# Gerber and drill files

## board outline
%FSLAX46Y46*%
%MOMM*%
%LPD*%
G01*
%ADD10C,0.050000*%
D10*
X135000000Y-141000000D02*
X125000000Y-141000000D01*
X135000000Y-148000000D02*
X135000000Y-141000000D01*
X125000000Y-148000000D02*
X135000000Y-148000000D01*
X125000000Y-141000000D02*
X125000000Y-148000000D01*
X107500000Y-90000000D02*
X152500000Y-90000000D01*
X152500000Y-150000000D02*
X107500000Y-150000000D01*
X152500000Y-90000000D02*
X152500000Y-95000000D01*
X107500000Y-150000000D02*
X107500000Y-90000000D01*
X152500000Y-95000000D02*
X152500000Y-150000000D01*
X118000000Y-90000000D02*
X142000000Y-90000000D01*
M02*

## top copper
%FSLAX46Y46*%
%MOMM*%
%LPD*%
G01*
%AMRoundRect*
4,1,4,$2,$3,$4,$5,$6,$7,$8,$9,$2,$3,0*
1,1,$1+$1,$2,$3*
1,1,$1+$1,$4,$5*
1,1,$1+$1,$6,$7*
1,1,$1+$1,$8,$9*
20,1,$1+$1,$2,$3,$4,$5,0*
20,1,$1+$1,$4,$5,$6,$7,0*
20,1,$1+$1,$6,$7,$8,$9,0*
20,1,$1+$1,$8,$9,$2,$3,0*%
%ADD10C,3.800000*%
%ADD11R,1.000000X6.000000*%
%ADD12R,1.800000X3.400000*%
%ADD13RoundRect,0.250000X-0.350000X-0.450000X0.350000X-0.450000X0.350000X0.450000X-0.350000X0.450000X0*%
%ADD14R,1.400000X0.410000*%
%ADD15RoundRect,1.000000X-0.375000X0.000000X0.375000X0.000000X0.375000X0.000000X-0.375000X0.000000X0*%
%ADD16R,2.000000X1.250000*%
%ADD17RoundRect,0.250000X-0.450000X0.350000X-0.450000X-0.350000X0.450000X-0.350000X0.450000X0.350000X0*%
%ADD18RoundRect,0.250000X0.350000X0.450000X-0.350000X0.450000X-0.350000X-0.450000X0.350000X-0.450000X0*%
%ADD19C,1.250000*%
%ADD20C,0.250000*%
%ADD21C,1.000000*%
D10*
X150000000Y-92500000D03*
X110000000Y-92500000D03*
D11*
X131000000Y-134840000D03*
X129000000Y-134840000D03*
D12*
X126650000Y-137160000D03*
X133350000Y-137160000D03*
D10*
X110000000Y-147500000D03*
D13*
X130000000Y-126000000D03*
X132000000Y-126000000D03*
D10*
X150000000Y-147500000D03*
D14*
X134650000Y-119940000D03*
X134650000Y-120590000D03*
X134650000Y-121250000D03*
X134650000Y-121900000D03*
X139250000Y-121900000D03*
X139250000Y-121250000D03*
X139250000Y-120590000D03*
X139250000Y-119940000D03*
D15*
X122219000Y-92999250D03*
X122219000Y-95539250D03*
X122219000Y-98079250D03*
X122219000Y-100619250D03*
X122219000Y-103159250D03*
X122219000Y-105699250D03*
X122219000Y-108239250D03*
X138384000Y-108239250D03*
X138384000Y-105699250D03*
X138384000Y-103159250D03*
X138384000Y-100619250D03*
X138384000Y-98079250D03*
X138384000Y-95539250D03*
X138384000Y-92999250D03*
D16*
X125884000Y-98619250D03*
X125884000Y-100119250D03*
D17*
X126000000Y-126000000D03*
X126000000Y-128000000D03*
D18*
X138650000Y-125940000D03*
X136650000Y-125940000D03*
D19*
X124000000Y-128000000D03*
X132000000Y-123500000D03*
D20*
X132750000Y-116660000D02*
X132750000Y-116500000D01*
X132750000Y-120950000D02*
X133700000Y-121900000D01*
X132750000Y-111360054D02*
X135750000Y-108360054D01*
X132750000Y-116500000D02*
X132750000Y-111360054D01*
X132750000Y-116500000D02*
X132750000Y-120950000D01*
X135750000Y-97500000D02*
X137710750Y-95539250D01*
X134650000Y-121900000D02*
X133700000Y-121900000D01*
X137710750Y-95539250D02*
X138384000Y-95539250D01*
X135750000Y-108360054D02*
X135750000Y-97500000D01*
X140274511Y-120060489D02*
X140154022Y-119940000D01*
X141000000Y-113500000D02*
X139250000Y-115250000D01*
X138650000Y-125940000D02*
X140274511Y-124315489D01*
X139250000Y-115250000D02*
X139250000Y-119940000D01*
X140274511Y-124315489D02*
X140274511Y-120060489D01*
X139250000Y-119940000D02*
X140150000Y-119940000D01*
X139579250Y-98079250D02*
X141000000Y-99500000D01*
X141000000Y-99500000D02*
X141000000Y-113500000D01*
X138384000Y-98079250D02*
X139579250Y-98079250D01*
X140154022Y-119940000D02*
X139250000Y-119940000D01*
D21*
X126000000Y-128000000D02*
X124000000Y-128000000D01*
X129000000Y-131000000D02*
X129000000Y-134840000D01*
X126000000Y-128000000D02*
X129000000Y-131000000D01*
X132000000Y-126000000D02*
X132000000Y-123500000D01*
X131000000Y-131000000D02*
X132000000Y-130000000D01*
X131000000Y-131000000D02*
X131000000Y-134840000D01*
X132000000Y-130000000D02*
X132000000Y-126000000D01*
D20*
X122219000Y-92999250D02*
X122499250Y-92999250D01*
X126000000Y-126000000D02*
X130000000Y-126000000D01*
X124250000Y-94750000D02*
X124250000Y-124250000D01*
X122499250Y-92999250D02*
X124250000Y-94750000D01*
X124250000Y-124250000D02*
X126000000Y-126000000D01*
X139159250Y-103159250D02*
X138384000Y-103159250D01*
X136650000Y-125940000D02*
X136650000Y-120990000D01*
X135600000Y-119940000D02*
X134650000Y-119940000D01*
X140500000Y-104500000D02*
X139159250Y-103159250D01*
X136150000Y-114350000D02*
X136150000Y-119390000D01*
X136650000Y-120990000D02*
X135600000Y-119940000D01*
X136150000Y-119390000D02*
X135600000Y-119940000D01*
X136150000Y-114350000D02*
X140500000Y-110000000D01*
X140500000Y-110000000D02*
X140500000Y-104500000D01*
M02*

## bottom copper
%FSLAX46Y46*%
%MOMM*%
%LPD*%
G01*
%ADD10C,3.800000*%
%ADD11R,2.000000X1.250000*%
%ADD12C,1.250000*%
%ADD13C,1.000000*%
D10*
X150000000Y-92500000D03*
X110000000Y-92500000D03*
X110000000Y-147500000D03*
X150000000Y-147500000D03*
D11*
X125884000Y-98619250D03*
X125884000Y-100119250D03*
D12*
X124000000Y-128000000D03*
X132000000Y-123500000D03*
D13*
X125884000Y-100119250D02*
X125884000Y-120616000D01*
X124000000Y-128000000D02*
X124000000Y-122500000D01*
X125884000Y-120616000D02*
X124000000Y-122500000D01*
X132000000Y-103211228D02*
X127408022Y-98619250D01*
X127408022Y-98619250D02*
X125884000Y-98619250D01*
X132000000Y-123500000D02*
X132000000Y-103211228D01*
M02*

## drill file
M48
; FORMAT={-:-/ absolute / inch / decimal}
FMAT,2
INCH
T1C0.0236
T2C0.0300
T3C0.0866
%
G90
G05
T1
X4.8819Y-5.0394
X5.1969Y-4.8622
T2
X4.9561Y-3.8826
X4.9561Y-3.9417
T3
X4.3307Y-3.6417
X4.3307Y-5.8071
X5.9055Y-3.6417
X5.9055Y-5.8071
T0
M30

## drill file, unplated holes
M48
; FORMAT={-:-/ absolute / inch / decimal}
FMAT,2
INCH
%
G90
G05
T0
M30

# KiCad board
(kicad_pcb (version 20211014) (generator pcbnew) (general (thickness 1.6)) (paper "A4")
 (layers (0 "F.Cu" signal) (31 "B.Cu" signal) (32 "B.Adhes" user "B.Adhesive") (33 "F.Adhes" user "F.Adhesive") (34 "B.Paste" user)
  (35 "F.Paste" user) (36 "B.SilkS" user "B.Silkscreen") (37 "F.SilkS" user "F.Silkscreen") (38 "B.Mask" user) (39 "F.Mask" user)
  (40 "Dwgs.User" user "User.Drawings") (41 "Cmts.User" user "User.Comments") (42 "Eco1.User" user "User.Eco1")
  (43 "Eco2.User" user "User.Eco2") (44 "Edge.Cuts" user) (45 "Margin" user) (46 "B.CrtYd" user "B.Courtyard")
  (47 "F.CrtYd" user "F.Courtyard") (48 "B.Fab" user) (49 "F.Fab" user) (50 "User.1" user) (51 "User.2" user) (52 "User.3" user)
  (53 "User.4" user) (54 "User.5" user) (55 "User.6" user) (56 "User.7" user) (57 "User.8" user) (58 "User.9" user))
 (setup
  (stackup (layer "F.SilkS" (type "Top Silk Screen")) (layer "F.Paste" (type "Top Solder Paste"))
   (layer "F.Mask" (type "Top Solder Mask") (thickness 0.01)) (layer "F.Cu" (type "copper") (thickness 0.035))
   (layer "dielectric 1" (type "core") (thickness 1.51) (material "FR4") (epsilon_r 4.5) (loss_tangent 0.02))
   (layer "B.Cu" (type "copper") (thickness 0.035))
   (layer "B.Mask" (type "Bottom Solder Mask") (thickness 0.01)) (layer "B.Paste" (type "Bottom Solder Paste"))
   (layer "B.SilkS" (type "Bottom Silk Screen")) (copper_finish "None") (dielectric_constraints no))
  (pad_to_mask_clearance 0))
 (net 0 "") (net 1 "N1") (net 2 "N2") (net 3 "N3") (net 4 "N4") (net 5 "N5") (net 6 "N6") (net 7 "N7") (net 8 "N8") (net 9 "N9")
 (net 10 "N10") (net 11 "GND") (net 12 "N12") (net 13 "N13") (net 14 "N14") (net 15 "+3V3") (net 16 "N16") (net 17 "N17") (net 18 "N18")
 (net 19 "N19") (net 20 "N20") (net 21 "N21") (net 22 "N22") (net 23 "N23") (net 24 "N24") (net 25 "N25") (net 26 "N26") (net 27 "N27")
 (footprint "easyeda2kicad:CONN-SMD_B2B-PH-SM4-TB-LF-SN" (layer "F.Cu") (at 130 136)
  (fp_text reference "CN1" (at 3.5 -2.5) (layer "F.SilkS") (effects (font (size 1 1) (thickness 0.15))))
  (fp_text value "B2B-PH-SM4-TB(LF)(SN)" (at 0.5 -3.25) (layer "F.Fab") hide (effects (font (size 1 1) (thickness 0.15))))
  (pad "1" smd rect locked (at 1 -1.16) (size 1 6) (layers "F.Cu" "F.Paste" "F.Mask") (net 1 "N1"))
  (pad "2" smd rect locked (at -1 -1.16) (size 1 6) (layers "F.Cu" "F.Paste" "F.Mask") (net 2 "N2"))
  (pad "3" smd rect locked (at -3.35 1.16) (size 1.8 3.4) (layers "F.Cu" "F.Paste" "F.Mask") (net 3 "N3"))
  (pad "4" smd rect locked (at 3.35 1.16) (size 1.8 3.4) (layers "F.Cu" "F.Paste" "F.Mask") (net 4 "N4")))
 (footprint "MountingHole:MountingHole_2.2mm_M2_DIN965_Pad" (layer "F.Cu") (at 110 147.5)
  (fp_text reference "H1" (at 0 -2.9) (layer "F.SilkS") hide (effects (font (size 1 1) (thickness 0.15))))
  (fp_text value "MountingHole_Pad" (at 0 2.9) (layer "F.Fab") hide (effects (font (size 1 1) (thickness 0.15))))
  (pad "1" thru_hole circle (at 0 0) (size 3.8 3.8) (drill 2.2) (layers *.Cu *.Mask) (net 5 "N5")))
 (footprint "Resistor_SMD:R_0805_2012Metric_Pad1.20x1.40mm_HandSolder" (layer "F.Cu") (at 131 126)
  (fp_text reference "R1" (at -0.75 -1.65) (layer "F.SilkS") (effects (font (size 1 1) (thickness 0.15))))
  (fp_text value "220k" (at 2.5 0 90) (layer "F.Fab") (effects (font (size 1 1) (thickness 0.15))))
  (pad "1" smd roundrect (at -1 0) (size 1.2 1.4) (layers "F.Cu" "F.Paste" "F.Mask") (roundrect_rratio 0.208333) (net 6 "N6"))
  (pad "2" smd roundrect (at 1 0) (size 1.2 1.4) (layers "F.Cu" "F.Paste" "F.Mask") (roundrect_rratio 0.208333) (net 1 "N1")))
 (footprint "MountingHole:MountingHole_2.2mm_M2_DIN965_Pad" (layer "F.Cu") (at 150 147.5)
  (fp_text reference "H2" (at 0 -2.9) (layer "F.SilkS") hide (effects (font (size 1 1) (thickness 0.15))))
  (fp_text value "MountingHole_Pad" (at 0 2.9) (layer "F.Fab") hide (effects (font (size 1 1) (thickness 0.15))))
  (pad "1" thru_hole circle (at 0 0) (size 3.8 3.8) (drill 2.2) (layers *.Cu *.Mask) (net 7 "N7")))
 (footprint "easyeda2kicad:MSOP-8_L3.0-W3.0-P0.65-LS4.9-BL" (layer "F.Cu") (at 136.95 120.92 -90)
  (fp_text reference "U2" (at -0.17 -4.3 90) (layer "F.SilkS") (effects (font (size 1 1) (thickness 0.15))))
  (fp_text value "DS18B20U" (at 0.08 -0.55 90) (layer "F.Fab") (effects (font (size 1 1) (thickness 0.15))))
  (pad "1" smd rect locked (at -0.98 2.3 270) (size 0.41 1.4) (layers "F.Cu" "F.Paste" "F.Mask") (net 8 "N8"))
  (pad "2" smd rect locked (at -0.33 2.3 270) (size 0.41 1.4) (layers "F.Cu" "F.Paste" "F.Mask") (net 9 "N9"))
  (pad "3" smd rect locked (at 0.33 2.3 270) (size 0.41 1.4) (layers "F.Cu" "F.Paste" "F.Mask") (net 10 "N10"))
  (pad "4" smd rect locked (at 0.98 2.3 270) (size 0.41 1.4) (layers "F.Cu" "F.Paste" "F.Mask") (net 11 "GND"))
  (pad "5" smd rect locked (at 0.98 -2.3 270) (size 0.41 1.4) (layers "F.Cu" "F.Paste" "F.Mask") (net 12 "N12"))
  (pad "6" smd rect locked (at 0.33 -2.3 270) (size 0.41 1.4) (layers "F.Cu" "F.Paste" "F.Mask") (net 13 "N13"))
  (pad "7" smd rect locked (at -0.33 -2.3 270) (size 0.41 1.4) (layers "F.Cu" "F.Paste" "F.Mask") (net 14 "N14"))
  (pad "8" smd rect locked (at -0.98 -2.3 270) (size 0.41 1.4) (layers "F.Cu" "F.Paste" "F.Mask") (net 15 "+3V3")))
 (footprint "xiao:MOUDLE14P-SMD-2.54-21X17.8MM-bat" (layer "F.Cu") (at 121.384 111.11925)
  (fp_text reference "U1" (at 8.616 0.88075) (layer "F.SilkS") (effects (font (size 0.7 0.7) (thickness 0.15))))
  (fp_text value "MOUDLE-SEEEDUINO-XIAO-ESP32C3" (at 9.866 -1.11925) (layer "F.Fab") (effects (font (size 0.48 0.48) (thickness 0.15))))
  (pad "1" smd roundrect (at 0.835 -18.12) (size 2.75 2) (layers "F.Cu" "F.Paste" "F.Mask") (roundrect_rratio 0.5) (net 6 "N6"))
  (pad "2" smd roundrect (at 0.835 -15.58) (size 2.75 2) (layers "F.Cu" "F.Paste" "F.Mask") (roundrect_rratio 0.5) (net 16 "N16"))
  (pad "3" smd roundrect (at 0.835 -13.04) (size 2.75 2) (layers "F.Cu" "F.Paste" "F.Mask") (roundrect_rratio 0.5) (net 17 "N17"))
  (pad "4" smd roundrect (at 0.835 -10.5) (size 2.75 2) (layers "F.Cu" "F.Paste" "F.Mask") (roundrect_rratio 0.5) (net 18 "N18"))
  (pad "5" smd roundrect (at 0.835 -7.96) (size 2.75 2) (layers "F.Cu" "F.Paste" "F.Mask") (roundrect_rratio 0.5) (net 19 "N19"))
  (pad "6" smd roundrect (at 0.835 -5.42) (size 2.75 2) (layers "F.Cu" "F.Paste" "F.Mask") (roundrect_rratio 0.5) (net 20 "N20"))
  (pad "7" smd roundrect (at 0.835 -2.88) (size 2.75 2) (layers "F.Cu" "F.Paste" "F.Mask") (roundrect_rratio 0.5) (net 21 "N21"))
  (pad "8" smd roundrect (at 17 -2.88) (size 2.75 2) (layers "F.Cu" "F.Paste" "F.Mask") (roundrect_rratio 0.5) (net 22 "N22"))
  (pad "9" smd roundrect (at 17 -5.42) (size 2.75 2) (layers "F.Cu" "F.Paste" "F.Mask") (roundrect_rratio 0.5) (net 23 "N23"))
  (pad "10" smd roundrect (at 17 -7.96) (size 2.75 2) (layers "F.Cu" "F.Paste" "F.Mask") (roundrect_rratio 0.5) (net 8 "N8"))
  (pad "11" smd roundrect (at 17 -10.5) (size 2.75 2) (layers "F.Cu" "F.Paste" "F.Mask") (roundrect_rratio 0.5) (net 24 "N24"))
  (pad "12" smd roundrect (at 17 -13.04) (size 2.75 2) (layers "F.Cu" "F.Paste" "F.Mask") (roundrect_rratio 0.5) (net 15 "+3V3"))
  (pad "13" smd roundrect (at 17 -15.58) (size 2.75 2) (layers "F.Cu" "F.Paste" "F.Mask") (roundrect_rratio 0.5) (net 11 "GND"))
  (pad "14" smd roundrect (at 17 -18.12) (size 2.75 2) (layers "F.Cu" "F.Paste" "F.Mask") (roundrect_rratio 0.5) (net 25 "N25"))
  (pad "15" thru_hole rect (at 4.5 -12.5) (size 2 1.25) (drill 0.762) (layers *.Cu *.Mask) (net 1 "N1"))
  (pad "16" thru_hole rect (at 4.5 -11) (size 2 1.25) (drill 0.762) (layers *.Cu *.Mask) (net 2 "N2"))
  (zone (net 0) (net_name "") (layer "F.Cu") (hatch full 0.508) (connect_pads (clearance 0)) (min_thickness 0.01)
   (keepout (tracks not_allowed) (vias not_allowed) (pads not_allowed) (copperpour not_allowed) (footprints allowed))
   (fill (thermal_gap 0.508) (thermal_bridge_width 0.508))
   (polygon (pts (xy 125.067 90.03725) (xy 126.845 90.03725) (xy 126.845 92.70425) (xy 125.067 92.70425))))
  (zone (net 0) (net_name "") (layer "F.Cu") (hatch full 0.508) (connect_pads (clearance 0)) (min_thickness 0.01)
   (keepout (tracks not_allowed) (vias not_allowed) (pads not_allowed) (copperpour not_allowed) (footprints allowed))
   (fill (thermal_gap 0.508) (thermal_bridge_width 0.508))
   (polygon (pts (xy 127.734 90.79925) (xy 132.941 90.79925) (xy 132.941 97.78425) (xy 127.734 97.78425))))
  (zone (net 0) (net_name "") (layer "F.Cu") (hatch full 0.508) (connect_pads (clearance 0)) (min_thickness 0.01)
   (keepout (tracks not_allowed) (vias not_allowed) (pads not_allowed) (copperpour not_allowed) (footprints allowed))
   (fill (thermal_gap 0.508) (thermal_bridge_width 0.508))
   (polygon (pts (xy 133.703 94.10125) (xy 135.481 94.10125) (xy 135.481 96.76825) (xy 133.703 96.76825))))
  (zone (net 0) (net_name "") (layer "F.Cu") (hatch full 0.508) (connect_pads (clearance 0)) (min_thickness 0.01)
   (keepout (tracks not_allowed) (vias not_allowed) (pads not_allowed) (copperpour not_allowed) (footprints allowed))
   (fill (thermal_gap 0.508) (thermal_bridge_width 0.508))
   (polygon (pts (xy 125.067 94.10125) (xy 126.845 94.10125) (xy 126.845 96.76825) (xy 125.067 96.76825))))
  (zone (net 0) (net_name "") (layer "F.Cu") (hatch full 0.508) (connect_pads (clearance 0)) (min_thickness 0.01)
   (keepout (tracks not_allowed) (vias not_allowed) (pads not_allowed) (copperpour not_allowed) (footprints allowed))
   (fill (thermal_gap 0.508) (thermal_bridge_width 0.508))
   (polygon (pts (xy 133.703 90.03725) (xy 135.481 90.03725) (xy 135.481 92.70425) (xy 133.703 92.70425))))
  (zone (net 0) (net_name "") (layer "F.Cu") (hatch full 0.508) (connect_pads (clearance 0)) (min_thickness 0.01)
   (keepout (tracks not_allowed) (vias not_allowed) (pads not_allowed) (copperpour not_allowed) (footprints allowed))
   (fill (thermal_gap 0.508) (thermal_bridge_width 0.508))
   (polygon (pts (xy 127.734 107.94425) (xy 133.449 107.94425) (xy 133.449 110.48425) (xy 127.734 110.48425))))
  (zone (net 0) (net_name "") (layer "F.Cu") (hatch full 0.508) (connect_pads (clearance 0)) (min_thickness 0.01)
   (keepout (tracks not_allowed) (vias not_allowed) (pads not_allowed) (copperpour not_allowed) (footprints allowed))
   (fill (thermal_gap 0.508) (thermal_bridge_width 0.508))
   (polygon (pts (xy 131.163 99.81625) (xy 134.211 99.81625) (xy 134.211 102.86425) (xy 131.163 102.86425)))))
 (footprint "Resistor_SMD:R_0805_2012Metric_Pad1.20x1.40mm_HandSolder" (layer "F.Cu") (at 126 127 -90)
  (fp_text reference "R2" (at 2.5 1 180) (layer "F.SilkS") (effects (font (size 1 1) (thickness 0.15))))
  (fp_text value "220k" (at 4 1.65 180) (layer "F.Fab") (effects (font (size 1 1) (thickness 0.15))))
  (pad "1" smd roundrect (at -1 0 270) (size 1.2 1.4) (layers "F.Cu" "F.Paste" "F.Mask") (roundrect_rratio 0.208333) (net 6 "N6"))
  (pad "2" smd roundrect (at 1 0 270) (size 1.2 1.4) (layers "F.Cu" "F.Paste" "F.Mask") (roundrect_rratio 0.208333) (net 2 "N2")))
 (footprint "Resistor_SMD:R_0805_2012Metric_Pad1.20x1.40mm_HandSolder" (layer "F.Cu") (at 137.65 125.94 180)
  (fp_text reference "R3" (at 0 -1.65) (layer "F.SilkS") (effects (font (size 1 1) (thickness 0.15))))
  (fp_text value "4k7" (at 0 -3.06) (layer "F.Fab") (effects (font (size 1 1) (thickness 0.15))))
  (pad "1" smd roundrect (at -1 0 180) (size 1.2 1.4) (layers "F.Cu" "F.Paste" "F.Mask") (roundrect_rratio 0.208333) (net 15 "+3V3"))
  (pad "2" smd roundrect (at 1 0 180) (size 1.2 1.4) (layers "F.Cu" "F.Paste" "F.Mask") (roundrect_rratio 0.208333) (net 8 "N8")))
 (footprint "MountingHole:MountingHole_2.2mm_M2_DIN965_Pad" (layer "F.Cu") (at 150 92.5)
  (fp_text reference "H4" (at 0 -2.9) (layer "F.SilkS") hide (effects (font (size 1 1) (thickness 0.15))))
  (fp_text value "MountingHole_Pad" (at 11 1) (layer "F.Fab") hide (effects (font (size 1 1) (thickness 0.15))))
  (pad "1" thru_hole circle (at 0 0) (size 3.8 3.8) (drill 2.2) (layers *.Cu *.Mask) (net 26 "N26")))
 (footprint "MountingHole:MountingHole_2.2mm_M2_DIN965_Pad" (layer "F.Cu") (at 110 92.5)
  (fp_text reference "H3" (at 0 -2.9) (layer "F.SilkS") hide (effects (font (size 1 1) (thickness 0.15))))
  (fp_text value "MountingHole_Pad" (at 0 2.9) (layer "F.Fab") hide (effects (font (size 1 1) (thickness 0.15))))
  (pad "1" thru_hole circle (at 0 0) (size 3.8 3.8) (drill 2.2) (layers *.Cu *.Mask) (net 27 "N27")))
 (gr_line (start 135 141) (end 125 141) (layer "Edge.Cuts") (width 0.05))
 (gr_line (start 107.5 90) (end 152.5 90) (layer "Edge.Cuts") (width 0.05))
 (gr_line (start 118 90) (end 142 90) (layer "Edge.Cuts") (width 0.05))
 (gr_line (start 125 148) (end 135 148) (layer "Edge.Cuts") (width 0.05))
 (gr_line (start 125 141) (end 125 148) (layer "Edge.Cuts") (width 0.05))
 (gr_line (start 107.5 150) (end 107.5 90) (layer "Edge.Cuts") (width 0.05))
 (gr_line (start 152.5 95) (end 152.5 150) (layer "Edge.Cuts") (width 0.05))
 (gr_line (start 135 148) (end 135 141) (layer "Edge.Cuts") (width 0.05))
 (gr_line (start 152.5 90) (end 152.5 95) (layer "Edge.Cuts") (width 0.05))
 (gr_line (start 152.5 150) (end 107.5 150) (layer "Edge.Cuts") (width 0.05))
 (segment (start 132.75 116.66) (end 132.75 116.5) (width 0.25) (layer "F.Cu") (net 11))
 (segment (start 132.75 120.95) (end 133.7 121.9) (width 0.25) (layer "F.Cu") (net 11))
 (segment (start 132.75 111.360054) (end 135.75 108.360054) (width 0.25) (layer "F.Cu") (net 11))
 (segment (start 132.75 116.5) (end 132.75 111.360054) (width 0.25) (layer "F.Cu") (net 11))
 (segment (start 132.75 116.5) (end 132.75 120.95) (width 0.25) (layer "F.Cu") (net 11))
 (segment (start 135.75 97.5) (end 137.71075 95.53925) (width 0.25) (layer "F.Cu") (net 11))
 (segment (start 134.65 121.9) (end 133.7 121.9) (width 0.25) (layer "F.Cu") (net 11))
 (segment (start 137.71075 95.53925) (end 138.384 95.53925) (width 0.25) (layer "F.Cu") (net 11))
 (segment (start 135.75 108.360054) (end 135.75 97.5) (width 0.25) (layer "F.Cu") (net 11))
 (segment (start 140.274511 120.060489) (end 140.154022 119.94) (width 0.25) (layer "F.Cu") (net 15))
 (segment (start 141 113.5) (end 139.25 115.25) (width 0.25) (layer "F.Cu") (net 15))
 (segment (start 138.65 125.94) (end 140.274511 124.315489) (width 0.25) (layer "F.Cu") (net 15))
 (segment (start 139.25 115.25) (end 139.25 119.94) (width 0.25) (layer "F.Cu") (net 15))
 (segment (start 140.274511 124.315489) (end 140.274511 120.060489) (width 0.25) (layer "F.Cu") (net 15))
 (segment (start 139.25 119.94) (end 140.15 119.94) (width 0.25) (layer "F.Cu") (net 15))
 (segment (start 139.57925 98.07925) (end 141 99.5) (width 0.25) (layer "F.Cu") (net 15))
 (segment (start 141 99.5) (end 141 113.5) (width 0.25) (layer "F.Cu") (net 15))
 (segment (start 138.384 98.07925) (end 139.57925 98.07925) (width 0.25) (layer "F.Cu") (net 15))
 (segment (start 140.154022 119.94) (end 139.25 119.94) (width 0.25) (layer "F.Cu") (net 15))
 (segment (start 126 128) (end 124 128) (width 1) (layer "F.Cu") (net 2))
 (segment (start 129 131) (end 129 134.84) (width 1) (layer "F.Cu") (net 2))
 (segment (start 126 128) (end 129 131) (width 1) (layer "F.Cu") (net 2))
 (via (at 124 128) (size 1.25) (drill 0.6) (layers "F.Cu" "B.Cu") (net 2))
 (segment (start 125.884 100.11925) (end 125.884 120.616) (width 1) (layer "B.Cu") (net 2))
 (segment (start 124 128) (end 124 122.5) (width 1) (layer "B.Cu") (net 2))
 (segment (start 125.884 120.616) (end 124 122.5) (width 1) (layer "B.Cu") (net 2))
 (segment (start 132 126) (end 132 123.5) (width 1) (layer "F.Cu") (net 1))
 (segment (start 131 131) (end 132 130) (width 1) (layer "F.Cu") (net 1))
 (segment (start 131 131) (end 131 134.84) (width 1) (layer "F.Cu") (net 1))
 (segment (start 132 130) (end 132 126) (width 1) (layer "F.Cu") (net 1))
 (via (at 132 123.5) (size 1.25) (drill 0.6) (layers "F.Cu" "B.Cu") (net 1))
 (segment (start 132 103.211228) (end 127.408022 98.61925) (width 1) (layer "B.Cu") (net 1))
 (segment (start 127.408022 98.61925) (end 125.884 98.61925) (width 1) (layer "B.Cu") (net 1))
 (segment (start 132 123.5) (end 132 103.211228) (width 1) (layer "B.Cu") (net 1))
 (segment (start 122.219 92.99925) (end 122.49925 92.99925) (width 0.25) (layer "F.Cu") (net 6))
 (segment (start 126 126) (end 130 126) (width 0.25) (layer "F.Cu") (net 6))
 (segment (start 124.25 94.75) (end 124.25 124.25) (width 0.25) (layer "F.Cu") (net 6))
 (segment (start 122.49925 92.99925) (end 124.25 94.75) (width 0.25) (layer "F.Cu") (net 6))
 (segment (start 124.25 124.25) (end 126 126) (width 0.25) (layer "F.Cu") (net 6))
 (segment (start 139.15925 103.15925) (end 138.384 103.15925) (width 0.25) (layer "F.Cu") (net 8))
 (segment (start 136.65 125.94) (end 136.65 120.99) (width 0.25) (layer "F.Cu") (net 8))
 (segment (start 135.6 119.94) (end 134.65 119.94) (width 0.25) (layer "F.Cu") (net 8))
 (segment (start 140.5 104.5) (end 139.15925 103.15925) (width 0.25) (layer "F.Cu") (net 8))
 (segment (start 136.15 114.35) (end 136.15 119.39) (width 0.25) (layer "F.Cu") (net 8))
 (segment (start 136.65 120.99) (end 135.6 119.94) (width 0.25) (layer "F.Cu") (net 8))
 (segment (start 136.15 119.39) (end 135.6 119.94) (width 0.25) (layer "F.Cu") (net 8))
 (segment (start 136.15 114.35) (end 140.5 110) (width 0.25) (layer "F.Cu") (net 8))
 (segment (start 140.5 110) (end 140.5 104.5) (width 0.25) (layer "F.Cu") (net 8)))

